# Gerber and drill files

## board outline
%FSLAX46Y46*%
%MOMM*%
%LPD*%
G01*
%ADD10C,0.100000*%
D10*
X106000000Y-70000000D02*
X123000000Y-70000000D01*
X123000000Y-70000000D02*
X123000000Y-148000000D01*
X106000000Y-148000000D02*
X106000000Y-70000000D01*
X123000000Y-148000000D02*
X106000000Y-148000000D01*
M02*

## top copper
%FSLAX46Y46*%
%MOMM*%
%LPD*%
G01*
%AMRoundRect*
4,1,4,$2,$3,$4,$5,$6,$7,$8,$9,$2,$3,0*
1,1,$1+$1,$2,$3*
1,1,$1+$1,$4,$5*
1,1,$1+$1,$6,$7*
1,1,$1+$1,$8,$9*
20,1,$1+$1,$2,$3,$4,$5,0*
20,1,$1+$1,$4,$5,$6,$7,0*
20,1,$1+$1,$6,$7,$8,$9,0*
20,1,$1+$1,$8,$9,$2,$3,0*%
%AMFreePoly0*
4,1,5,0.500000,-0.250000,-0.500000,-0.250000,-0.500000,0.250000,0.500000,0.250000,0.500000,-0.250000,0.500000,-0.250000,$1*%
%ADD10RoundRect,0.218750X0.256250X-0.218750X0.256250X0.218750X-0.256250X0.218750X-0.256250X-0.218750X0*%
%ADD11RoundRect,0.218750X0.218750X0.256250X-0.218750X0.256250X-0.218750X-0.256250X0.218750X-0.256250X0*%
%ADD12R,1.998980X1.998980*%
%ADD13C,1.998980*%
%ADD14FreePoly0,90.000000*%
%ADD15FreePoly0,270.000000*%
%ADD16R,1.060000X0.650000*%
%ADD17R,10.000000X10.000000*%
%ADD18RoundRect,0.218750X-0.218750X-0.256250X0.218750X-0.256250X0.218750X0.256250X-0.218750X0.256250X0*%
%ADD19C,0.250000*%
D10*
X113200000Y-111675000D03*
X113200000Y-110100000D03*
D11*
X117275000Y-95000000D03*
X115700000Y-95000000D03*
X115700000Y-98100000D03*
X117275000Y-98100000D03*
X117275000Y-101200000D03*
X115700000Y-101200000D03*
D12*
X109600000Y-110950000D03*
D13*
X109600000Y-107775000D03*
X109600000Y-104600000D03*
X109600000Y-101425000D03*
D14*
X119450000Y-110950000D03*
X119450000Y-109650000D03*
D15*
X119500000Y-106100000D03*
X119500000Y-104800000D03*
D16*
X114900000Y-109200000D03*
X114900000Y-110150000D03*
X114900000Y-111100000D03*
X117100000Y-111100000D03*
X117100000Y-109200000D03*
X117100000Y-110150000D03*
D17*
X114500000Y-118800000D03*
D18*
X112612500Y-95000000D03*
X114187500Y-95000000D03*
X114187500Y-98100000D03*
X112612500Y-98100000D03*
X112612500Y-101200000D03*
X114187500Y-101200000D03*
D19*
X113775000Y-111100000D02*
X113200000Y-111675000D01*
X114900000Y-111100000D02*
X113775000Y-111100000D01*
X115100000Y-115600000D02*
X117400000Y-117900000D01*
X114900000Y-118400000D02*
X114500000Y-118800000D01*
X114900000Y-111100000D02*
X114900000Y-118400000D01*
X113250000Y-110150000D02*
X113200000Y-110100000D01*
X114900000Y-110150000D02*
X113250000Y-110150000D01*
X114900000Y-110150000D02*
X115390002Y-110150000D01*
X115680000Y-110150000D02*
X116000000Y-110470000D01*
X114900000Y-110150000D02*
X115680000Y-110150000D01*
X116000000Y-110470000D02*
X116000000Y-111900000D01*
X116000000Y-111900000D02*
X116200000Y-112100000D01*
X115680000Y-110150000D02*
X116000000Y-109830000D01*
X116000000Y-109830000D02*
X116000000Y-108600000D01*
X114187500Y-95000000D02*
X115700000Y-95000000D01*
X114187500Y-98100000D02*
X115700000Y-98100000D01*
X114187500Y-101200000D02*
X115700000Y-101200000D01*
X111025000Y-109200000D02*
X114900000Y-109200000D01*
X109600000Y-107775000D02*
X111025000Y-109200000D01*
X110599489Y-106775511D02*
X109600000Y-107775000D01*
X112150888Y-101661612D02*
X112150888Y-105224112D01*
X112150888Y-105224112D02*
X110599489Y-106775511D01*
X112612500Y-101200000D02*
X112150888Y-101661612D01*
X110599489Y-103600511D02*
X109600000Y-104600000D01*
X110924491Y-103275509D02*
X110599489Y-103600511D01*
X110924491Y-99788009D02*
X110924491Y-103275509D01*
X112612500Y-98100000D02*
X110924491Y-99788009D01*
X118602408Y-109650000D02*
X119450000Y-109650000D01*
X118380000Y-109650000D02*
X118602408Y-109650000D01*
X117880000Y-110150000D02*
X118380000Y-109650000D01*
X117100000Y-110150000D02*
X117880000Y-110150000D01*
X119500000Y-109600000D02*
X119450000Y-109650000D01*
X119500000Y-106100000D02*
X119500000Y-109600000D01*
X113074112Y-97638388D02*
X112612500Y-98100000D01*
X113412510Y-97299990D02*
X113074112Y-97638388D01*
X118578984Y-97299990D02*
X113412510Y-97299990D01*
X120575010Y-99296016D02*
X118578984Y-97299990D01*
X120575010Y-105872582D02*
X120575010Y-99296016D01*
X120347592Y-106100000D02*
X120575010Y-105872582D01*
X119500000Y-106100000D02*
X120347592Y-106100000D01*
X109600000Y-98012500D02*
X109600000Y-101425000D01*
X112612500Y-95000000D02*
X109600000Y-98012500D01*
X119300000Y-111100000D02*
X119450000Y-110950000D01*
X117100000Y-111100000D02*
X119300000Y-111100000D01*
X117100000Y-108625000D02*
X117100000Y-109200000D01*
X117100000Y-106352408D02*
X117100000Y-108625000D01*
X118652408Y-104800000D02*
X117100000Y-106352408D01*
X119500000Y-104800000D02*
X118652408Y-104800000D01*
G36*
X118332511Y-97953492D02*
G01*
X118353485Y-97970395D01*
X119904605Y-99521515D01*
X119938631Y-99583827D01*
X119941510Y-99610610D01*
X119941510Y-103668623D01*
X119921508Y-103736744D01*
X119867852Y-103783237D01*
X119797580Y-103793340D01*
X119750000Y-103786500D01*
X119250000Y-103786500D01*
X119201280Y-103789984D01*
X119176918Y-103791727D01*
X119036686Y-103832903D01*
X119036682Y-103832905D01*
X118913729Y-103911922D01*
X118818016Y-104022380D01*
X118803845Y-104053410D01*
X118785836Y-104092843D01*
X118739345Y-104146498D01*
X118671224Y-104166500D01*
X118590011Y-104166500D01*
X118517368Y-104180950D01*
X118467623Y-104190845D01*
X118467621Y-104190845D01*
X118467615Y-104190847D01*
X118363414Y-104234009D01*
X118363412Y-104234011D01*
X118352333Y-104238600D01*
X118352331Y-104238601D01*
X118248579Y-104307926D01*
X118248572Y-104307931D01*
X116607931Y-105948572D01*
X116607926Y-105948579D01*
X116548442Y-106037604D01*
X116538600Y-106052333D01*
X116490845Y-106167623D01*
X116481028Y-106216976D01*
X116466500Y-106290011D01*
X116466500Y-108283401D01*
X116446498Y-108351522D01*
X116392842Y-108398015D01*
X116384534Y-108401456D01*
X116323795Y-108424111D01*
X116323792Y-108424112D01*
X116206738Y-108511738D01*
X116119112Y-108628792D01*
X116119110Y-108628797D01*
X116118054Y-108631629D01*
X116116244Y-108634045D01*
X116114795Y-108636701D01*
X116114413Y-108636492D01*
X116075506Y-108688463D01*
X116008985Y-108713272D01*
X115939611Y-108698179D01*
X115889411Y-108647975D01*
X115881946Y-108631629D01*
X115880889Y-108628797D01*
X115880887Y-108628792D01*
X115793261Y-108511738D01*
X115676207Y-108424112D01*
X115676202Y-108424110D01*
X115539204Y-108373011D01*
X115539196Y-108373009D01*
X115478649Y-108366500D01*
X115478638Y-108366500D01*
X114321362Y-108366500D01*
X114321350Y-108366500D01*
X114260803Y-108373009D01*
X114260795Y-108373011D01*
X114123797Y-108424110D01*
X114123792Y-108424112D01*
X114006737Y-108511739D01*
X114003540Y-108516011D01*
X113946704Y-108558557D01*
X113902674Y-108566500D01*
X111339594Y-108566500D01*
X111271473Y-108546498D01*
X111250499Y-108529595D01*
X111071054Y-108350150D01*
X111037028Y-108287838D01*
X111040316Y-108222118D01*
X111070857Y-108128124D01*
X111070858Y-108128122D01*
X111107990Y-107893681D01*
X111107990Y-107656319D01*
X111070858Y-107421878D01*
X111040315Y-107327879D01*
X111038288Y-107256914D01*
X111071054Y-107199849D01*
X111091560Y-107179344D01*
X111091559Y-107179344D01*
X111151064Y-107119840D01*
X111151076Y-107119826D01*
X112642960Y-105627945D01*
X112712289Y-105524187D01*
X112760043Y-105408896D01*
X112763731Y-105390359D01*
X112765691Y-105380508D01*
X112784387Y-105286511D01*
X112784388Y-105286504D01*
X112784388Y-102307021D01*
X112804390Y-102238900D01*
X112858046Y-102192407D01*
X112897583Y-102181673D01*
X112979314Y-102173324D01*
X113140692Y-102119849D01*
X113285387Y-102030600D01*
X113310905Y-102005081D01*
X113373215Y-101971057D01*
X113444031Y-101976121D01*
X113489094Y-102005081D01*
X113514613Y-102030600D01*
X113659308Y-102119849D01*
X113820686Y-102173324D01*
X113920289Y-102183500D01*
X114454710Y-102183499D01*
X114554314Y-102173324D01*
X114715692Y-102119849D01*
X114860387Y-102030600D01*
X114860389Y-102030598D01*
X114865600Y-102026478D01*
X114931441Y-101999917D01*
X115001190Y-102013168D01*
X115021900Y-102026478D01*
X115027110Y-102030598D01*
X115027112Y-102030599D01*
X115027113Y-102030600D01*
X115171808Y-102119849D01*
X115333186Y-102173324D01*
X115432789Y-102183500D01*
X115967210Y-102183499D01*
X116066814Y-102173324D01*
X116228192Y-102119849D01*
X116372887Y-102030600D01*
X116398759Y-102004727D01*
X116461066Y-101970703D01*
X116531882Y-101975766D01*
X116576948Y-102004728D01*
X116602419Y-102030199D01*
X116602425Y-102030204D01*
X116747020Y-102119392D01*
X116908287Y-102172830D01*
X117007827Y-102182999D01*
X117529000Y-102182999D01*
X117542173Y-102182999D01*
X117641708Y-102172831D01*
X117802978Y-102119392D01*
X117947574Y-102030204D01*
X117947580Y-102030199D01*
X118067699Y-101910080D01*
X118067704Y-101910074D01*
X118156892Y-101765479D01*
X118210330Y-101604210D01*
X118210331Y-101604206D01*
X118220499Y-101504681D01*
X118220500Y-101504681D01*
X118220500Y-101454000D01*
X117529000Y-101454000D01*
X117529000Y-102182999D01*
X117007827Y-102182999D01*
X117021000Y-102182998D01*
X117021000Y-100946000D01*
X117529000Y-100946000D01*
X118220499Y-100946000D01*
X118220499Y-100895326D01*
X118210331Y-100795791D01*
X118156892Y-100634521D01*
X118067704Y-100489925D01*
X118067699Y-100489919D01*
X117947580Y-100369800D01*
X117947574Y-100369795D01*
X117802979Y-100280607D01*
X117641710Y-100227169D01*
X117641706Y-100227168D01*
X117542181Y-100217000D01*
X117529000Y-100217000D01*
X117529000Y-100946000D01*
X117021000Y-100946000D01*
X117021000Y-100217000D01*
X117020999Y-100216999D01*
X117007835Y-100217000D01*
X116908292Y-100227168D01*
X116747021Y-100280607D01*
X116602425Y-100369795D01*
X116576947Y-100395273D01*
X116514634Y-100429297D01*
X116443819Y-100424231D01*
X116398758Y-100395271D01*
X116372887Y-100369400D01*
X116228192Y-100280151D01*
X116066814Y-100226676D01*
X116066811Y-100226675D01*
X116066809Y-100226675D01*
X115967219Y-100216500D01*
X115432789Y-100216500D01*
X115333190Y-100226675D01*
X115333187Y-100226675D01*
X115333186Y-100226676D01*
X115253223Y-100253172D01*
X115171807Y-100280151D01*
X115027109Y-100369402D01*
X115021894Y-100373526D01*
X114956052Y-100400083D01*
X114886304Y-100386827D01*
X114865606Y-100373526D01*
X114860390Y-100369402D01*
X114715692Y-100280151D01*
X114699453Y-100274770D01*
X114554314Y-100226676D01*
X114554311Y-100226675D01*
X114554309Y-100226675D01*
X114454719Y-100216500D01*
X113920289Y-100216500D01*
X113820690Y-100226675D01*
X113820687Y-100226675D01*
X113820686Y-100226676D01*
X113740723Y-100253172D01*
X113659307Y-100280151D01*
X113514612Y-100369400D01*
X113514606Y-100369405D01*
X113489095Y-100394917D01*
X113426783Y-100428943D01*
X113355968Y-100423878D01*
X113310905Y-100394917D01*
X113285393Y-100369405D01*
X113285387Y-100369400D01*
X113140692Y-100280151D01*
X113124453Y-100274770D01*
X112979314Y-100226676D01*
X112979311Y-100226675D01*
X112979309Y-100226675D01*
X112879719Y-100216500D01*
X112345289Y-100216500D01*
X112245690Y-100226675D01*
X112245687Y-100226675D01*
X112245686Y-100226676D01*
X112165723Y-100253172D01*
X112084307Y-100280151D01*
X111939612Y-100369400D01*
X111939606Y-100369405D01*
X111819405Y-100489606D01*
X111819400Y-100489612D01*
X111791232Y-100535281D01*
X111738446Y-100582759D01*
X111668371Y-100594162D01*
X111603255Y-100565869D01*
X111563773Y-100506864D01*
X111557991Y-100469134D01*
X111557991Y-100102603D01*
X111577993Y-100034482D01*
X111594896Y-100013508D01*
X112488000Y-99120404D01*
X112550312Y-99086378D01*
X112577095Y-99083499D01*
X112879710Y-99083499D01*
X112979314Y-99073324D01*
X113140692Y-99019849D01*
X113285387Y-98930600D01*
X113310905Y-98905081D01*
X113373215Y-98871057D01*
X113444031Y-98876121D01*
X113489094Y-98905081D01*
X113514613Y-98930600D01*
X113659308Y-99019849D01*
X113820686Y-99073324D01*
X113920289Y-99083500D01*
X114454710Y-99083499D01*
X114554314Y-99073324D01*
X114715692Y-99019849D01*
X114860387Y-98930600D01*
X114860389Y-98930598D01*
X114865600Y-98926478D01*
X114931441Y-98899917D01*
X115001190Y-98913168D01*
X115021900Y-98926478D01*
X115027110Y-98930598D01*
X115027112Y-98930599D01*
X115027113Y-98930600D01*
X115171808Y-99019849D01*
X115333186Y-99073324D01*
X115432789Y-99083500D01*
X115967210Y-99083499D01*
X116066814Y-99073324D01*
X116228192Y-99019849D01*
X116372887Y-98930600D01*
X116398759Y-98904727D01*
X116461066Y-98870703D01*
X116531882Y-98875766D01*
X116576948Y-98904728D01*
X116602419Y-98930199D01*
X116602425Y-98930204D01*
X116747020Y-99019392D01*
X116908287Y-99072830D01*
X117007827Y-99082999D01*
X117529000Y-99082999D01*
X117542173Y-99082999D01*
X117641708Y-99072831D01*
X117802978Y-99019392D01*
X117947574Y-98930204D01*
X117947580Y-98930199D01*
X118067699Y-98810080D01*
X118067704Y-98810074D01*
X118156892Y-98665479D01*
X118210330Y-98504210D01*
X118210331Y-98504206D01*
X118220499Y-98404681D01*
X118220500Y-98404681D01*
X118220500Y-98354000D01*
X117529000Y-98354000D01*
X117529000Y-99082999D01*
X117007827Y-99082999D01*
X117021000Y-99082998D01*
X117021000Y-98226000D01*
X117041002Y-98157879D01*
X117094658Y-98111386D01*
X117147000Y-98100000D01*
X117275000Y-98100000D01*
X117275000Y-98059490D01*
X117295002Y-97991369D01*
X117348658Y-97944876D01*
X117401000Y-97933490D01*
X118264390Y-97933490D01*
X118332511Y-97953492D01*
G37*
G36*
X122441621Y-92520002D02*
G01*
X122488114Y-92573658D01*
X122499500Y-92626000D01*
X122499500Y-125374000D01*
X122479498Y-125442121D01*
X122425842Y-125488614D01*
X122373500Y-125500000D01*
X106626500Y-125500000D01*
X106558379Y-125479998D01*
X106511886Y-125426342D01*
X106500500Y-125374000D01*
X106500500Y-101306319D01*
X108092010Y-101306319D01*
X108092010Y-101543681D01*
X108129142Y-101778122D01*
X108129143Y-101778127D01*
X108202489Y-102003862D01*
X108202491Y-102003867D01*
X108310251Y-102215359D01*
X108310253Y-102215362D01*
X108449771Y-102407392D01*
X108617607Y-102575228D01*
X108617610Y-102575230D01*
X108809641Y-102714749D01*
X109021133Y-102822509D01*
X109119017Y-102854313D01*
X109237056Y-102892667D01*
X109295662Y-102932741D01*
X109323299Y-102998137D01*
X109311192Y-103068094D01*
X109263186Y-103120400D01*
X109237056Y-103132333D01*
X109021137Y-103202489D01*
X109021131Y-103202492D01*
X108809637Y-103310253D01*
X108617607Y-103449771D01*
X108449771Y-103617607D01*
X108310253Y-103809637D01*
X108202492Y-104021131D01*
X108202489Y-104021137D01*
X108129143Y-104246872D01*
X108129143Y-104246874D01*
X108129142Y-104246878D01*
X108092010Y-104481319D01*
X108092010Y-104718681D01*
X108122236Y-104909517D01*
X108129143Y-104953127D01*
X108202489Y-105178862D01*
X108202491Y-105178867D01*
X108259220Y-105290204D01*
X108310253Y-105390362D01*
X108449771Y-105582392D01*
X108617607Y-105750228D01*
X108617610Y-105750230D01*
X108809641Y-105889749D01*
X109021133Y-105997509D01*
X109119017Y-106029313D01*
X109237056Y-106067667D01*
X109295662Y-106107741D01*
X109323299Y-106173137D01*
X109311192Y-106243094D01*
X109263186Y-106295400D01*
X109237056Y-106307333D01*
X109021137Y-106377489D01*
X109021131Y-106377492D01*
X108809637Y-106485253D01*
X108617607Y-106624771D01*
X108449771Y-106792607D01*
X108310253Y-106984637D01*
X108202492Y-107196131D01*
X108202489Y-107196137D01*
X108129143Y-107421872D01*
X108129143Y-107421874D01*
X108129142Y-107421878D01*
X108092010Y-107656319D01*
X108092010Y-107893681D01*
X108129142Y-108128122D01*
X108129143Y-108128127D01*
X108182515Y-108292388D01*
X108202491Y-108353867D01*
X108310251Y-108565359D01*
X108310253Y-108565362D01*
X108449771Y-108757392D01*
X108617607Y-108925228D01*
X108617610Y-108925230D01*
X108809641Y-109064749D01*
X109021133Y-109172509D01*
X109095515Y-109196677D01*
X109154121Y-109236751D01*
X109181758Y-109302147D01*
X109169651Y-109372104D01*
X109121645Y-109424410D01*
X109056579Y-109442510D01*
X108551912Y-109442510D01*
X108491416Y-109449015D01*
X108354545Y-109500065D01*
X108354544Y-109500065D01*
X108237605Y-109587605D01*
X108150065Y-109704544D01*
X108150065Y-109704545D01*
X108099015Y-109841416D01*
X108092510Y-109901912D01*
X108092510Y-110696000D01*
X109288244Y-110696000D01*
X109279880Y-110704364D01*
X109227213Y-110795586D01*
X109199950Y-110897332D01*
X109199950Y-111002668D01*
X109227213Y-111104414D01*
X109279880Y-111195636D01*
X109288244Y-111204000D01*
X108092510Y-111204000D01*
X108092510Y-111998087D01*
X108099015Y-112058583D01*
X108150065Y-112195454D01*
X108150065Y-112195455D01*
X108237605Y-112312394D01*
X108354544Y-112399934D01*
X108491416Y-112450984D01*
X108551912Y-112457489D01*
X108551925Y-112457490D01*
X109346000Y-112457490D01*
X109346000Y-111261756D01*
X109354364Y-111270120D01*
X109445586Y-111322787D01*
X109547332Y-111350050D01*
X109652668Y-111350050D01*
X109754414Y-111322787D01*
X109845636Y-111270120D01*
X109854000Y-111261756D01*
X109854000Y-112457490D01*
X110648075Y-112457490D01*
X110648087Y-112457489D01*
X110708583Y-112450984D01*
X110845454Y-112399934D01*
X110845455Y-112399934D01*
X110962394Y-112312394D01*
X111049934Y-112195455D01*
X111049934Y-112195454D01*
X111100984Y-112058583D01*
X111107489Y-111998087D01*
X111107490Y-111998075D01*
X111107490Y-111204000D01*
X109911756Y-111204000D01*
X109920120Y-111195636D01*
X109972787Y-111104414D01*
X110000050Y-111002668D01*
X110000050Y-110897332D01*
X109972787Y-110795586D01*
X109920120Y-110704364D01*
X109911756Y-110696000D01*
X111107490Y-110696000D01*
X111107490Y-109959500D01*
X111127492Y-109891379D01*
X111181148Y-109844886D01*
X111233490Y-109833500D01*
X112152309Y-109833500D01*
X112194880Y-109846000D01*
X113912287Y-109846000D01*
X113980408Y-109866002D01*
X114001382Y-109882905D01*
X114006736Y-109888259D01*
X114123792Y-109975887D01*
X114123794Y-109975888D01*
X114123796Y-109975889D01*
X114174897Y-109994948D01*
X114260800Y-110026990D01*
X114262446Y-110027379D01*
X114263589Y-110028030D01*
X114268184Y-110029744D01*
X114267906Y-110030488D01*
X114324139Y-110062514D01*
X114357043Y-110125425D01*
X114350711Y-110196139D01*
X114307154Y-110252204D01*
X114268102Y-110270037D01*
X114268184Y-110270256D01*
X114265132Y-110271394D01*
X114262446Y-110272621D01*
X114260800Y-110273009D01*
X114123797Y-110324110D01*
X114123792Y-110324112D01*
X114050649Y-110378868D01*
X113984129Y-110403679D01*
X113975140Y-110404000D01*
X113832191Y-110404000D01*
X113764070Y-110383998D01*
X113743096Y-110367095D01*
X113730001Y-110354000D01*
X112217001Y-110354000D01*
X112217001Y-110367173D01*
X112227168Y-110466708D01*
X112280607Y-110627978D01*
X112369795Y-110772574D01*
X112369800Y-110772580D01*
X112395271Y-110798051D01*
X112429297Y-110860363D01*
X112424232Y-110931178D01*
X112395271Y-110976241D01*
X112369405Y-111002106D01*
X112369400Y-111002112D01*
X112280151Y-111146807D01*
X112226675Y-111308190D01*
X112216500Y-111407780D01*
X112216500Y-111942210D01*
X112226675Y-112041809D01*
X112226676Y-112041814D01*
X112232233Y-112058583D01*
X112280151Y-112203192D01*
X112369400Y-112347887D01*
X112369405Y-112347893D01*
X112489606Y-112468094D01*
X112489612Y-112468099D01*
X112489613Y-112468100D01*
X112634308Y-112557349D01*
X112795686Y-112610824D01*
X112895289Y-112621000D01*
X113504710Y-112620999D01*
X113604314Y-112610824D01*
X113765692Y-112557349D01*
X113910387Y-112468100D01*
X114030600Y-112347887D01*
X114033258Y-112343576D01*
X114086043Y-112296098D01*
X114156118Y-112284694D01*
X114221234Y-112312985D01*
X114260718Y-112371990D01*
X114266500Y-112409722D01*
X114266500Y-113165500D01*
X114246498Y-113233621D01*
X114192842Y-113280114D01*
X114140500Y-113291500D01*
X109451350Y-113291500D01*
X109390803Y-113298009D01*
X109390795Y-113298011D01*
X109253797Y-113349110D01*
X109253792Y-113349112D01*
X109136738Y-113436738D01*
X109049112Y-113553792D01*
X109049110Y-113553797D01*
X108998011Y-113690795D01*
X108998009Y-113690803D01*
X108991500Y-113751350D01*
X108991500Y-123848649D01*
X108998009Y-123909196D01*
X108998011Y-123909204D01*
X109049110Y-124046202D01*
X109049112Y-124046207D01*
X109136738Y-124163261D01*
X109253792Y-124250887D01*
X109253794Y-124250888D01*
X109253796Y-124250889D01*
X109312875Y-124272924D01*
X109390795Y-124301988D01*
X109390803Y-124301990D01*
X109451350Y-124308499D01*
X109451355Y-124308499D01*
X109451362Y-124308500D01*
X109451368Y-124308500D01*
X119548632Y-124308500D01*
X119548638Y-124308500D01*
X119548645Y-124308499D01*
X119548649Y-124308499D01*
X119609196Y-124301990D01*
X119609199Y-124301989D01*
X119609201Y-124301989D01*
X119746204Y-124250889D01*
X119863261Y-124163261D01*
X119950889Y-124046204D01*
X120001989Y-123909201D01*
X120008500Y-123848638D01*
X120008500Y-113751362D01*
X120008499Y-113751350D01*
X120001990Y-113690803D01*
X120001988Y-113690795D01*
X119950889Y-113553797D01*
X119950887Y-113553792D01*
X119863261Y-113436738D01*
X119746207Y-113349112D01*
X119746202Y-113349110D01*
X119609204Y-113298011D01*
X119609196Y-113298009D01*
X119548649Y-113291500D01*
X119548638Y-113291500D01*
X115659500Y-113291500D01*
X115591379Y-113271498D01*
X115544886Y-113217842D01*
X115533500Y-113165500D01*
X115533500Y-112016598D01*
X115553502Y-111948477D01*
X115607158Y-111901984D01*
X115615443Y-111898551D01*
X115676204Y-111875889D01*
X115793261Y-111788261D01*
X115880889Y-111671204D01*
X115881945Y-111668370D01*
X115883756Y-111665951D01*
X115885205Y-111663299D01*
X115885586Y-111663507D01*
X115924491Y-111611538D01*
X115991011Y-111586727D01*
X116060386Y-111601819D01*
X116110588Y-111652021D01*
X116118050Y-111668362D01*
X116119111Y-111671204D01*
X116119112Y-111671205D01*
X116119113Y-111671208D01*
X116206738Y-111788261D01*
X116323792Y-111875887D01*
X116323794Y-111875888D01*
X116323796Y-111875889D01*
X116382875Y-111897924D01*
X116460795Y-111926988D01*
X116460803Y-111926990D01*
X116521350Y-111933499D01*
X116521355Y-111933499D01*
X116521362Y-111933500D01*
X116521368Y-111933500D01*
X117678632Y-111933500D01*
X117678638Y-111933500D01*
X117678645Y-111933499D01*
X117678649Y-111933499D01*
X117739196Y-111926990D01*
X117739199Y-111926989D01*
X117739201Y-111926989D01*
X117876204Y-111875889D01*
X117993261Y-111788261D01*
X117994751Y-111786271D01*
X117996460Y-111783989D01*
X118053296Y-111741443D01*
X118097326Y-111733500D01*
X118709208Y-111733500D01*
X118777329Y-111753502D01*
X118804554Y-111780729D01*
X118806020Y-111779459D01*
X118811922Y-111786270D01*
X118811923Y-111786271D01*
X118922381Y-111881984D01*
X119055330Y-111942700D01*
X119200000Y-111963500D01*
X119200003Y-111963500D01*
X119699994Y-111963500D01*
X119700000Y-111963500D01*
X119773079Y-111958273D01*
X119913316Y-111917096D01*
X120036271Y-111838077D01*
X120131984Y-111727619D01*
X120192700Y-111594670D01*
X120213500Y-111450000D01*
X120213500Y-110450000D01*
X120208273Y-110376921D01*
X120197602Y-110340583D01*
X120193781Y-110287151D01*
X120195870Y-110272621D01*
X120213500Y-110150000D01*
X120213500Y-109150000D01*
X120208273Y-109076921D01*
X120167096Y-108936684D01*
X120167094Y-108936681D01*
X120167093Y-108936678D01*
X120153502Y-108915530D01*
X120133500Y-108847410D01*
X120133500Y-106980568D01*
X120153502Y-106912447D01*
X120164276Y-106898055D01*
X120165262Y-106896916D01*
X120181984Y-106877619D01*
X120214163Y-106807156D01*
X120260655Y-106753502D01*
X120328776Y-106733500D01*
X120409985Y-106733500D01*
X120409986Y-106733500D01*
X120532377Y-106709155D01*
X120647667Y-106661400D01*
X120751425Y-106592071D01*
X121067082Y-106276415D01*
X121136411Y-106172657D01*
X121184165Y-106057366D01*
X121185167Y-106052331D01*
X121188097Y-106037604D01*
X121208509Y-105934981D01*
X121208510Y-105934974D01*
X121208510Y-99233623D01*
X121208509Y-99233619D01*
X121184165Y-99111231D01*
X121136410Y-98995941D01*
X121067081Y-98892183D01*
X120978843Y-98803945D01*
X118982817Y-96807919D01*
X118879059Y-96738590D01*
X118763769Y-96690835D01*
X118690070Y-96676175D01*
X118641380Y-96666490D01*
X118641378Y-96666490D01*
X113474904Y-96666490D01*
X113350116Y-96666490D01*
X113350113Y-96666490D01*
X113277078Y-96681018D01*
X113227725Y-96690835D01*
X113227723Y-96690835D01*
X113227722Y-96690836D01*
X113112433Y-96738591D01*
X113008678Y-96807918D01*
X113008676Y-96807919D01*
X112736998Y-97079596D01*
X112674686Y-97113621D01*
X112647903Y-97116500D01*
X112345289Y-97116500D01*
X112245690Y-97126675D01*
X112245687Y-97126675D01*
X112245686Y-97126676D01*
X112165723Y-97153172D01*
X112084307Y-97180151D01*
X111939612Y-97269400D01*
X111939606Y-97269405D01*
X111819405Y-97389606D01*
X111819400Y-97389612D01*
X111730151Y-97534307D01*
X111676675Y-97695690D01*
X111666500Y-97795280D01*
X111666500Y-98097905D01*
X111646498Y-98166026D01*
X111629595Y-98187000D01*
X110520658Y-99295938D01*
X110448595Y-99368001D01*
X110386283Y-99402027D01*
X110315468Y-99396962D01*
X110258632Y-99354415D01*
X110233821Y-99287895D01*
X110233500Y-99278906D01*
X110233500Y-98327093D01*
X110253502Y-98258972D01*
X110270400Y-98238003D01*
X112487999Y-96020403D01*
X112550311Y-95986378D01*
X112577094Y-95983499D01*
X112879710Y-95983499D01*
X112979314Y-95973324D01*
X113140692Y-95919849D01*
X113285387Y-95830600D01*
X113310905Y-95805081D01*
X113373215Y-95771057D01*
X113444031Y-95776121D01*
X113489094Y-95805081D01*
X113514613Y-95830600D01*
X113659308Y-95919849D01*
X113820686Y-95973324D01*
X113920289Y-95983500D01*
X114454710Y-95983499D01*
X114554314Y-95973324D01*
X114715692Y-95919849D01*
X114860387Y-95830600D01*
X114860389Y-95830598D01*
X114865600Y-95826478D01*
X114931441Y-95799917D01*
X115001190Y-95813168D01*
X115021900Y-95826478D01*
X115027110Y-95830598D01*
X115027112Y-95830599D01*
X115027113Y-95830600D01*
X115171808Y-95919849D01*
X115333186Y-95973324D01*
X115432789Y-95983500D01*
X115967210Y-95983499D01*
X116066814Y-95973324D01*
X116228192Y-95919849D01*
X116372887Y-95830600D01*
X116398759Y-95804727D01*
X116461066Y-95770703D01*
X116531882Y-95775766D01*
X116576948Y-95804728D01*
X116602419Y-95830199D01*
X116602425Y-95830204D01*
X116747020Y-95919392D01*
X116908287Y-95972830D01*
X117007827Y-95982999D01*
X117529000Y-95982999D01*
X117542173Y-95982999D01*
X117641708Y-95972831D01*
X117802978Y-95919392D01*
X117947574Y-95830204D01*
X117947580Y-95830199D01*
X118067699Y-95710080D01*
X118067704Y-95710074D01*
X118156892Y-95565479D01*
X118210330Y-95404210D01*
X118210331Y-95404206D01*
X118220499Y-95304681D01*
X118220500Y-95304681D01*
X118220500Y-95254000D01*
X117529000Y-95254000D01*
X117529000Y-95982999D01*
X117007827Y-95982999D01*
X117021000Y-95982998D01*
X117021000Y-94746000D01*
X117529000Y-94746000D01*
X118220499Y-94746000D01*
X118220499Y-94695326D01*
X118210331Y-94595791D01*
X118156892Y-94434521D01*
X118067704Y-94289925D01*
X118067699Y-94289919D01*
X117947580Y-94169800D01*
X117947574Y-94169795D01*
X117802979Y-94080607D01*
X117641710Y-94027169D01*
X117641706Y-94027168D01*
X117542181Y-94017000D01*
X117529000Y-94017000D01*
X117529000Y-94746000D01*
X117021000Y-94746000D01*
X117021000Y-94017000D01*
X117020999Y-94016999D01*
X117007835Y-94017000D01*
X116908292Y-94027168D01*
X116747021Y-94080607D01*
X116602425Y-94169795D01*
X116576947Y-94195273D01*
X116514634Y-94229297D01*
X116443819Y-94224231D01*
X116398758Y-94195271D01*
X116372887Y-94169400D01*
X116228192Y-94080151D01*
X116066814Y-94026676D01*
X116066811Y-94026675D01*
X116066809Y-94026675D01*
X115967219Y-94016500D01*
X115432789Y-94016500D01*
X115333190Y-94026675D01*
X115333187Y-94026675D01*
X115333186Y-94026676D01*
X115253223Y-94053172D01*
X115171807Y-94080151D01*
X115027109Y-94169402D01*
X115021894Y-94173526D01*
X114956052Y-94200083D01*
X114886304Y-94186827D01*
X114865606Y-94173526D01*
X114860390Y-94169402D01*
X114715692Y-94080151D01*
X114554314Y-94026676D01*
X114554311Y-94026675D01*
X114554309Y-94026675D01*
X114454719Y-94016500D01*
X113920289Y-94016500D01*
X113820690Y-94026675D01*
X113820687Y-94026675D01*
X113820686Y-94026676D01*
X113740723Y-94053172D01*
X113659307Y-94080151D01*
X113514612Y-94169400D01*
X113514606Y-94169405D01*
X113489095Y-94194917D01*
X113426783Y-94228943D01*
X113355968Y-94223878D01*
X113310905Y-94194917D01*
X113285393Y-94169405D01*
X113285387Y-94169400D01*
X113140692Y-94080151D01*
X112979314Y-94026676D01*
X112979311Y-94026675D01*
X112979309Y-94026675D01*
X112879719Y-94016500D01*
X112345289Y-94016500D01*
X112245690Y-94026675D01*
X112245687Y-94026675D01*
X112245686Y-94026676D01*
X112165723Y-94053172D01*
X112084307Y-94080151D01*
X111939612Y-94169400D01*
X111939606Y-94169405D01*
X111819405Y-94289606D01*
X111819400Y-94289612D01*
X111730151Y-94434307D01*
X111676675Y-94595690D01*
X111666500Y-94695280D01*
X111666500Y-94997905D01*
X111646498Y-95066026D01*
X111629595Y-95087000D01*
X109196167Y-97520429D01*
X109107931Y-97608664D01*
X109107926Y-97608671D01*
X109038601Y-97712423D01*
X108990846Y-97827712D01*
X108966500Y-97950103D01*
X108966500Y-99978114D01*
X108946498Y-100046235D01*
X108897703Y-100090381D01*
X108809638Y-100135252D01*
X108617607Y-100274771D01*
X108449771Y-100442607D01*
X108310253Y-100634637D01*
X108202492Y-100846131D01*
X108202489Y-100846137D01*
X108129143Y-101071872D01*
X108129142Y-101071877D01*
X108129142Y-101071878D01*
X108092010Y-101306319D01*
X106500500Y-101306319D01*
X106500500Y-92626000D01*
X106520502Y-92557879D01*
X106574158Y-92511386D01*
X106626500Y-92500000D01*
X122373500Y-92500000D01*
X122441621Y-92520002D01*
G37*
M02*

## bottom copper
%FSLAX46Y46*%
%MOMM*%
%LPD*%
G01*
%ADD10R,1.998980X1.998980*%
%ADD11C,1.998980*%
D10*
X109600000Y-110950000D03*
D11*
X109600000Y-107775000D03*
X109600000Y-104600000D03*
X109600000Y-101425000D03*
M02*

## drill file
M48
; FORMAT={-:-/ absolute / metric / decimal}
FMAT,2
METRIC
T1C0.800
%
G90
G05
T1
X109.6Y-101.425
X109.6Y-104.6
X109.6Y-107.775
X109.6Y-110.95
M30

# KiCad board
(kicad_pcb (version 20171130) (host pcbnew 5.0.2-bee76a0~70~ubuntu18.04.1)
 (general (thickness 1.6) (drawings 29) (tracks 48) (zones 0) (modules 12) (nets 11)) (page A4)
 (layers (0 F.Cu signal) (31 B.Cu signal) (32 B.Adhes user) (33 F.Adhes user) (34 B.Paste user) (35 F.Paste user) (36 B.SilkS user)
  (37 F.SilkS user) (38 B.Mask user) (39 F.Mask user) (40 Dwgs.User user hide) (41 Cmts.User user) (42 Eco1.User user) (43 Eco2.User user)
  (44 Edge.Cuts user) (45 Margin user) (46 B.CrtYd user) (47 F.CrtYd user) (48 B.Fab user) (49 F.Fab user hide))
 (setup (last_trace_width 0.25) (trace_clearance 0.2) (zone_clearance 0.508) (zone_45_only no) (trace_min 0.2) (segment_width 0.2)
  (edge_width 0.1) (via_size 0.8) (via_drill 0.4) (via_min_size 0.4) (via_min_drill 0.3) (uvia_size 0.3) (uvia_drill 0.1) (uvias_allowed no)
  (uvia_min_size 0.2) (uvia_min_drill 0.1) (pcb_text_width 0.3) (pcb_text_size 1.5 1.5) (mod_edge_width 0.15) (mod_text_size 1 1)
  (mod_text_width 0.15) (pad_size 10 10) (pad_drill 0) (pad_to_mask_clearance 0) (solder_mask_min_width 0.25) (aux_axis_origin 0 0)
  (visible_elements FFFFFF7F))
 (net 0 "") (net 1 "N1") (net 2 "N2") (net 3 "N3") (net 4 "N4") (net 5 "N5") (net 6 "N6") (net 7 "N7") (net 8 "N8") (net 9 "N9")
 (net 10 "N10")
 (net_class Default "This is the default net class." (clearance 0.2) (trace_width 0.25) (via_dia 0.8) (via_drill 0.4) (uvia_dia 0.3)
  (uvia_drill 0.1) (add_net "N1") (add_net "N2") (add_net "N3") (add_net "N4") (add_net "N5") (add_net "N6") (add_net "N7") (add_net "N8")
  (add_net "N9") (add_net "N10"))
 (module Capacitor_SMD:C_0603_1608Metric (layer F.Cu) (at 113.2 110.8875 90)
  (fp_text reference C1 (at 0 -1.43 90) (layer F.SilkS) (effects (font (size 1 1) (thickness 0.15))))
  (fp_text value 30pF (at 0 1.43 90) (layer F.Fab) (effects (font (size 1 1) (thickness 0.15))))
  (pad 1 smd roundrect (at -0.7875 0 90) (size 0.875 0.95) (layers F.Cu F.Paste F.Mask) (roundrect_rratio 0.25) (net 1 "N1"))
  (pad 2 smd roundrect (at 0.7875 0 90) (size 0.875 0.95) (layers F.Cu F.Paste F.Mask) (roundrect_rratio 0.25) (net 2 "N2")))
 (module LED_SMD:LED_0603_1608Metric (layer F.Cu) (at 116.4875 95 180)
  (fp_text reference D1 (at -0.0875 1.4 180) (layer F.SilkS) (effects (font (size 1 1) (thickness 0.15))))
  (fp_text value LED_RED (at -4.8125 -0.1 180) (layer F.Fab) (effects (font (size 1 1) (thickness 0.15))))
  (pad 1 smd roundrect (at -0.7875 0 180) (size 0.875 0.95) (layers F.Cu F.Paste F.Mask) (roundrect_rratio 0.25) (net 2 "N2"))
  (pad 2 smd roundrect (at 0.7875 0 180) (size 0.875 0.95) (layers F.Cu F.Paste F.Mask) (roundrect_rratio 0.25) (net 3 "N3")))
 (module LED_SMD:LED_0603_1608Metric (layer F.Cu) (at 116.4875 98.1 180)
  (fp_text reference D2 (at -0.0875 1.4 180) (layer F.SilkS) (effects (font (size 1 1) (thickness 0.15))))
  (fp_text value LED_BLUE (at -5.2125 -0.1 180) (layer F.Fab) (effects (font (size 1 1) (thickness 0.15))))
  (pad 2 smd roundrect (at 0.7875 0 180) (size 0.875 0.95) (layers F.Cu F.Paste F.Mask) (roundrect_rratio 0.25) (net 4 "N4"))
  (pad 1 smd roundrect (at -0.7875 0 180) (size 0.875 0.95) (layers F.Cu F.Paste F.Mask) (roundrect_rratio 0.25) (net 2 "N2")))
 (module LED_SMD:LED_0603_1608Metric (layer F.Cu) (at 116.4875 101.2 180)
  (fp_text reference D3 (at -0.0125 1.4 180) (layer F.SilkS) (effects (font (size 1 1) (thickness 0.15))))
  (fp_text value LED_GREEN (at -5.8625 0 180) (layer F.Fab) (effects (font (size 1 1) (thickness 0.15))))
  (pad 1 smd roundrect (at -0.7875 0 180) (size 0.875 0.95) (layers F.Cu F.Paste F.Mask) (roundrect_rratio 0.25) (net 2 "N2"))
  (pad 2 smd roundrect (at 0.7875 0 180) (size 0.875 0.95) (layers F.Cu F.Paste F.Mask) (roundrect_rratio 0.25) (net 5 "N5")))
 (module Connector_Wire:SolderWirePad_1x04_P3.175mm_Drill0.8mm (layer F.Cu) (at 109.6 110.95 90)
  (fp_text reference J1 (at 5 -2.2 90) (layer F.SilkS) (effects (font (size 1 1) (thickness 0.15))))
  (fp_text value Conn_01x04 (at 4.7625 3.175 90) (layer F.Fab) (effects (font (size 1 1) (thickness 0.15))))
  (pad 1 thru_hole rect (at 0 0 90) (size 1.99898 1.99898) (drill 0.8001) (layers *.Cu *.Mask) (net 2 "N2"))
  (pad 2 thru_hole circle (at 3.175 0 90) (size 1.99898 1.99898) (drill 0.8001) (layers *.Cu *.Mask) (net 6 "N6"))
  (pad 3 thru_hole circle (at 6.35 0 90) (size 1.99898 1.99898) (drill 0.8001) (layers *.Cu *.Mask) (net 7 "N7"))
  (pad 4 thru_hole circle (at 9.525 0 90) (size 1.99898 1.99898) (drill 0.8001) (layers *.Cu *.Mask) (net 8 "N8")))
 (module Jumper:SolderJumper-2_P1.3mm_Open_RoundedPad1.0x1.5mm (layer F.Cu) (at 119.45 110.3 90)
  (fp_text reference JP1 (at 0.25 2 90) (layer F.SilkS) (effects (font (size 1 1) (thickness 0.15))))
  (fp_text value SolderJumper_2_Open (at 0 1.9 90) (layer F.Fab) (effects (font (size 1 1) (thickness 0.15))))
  (pad 1 smd custom (at -0.65 0 90) (size 1 0.5) (layers F.Cu F.Mask) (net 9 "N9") (zone_connect 0)
   (options (clearance outline) (anchor rect)) (primitives))
  (pad 2 smd custom (at 0.65 0 90) (size 1 0.5) (layers F.Cu F.Mask) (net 7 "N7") (zone_connect 0)
   (options (clearance outline) (anchor rect)) (primitives)))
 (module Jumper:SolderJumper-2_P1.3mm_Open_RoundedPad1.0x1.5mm (layer F.Cu) (at 119.5 105.45 270)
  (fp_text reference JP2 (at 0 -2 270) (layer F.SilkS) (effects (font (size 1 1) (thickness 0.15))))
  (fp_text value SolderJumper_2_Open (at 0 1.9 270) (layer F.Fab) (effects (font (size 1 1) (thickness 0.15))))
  (pad 2 smd custom (at 0.65 0 270) (size 1 0.5) (layers F.Cu F.Mask) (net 7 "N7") (zone_connect 0)
   (options (clearance outline) (anchor rect)) (primitives))
  (pad 1 smd custom (at -0.65 0 270) (size 1 0.5) (layers F.Cu F.Mask) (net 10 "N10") (zone_connect 0)
   (options (clearance outline) (anchor rect)) (primitives)))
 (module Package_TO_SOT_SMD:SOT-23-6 (layer F.Cu) (at 116 110.15)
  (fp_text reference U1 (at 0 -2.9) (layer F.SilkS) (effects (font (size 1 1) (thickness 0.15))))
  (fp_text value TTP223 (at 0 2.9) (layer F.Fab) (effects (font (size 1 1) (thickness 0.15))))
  (pad 1 smd rect (at -1.1 -0.95) (size 1.06 0.65) (layers F.Cu F.Paste F.Mask) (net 6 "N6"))
  (pad 2 smd rect (at -1.1 0) (size 1.06 0.65) (layers F.Cu F.Paste F.Mask) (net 2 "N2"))
  (pad 3 smd rect (at -1.1 0.95) (size 1.06 0.65) (layers F.Cu F.Paste F.Mask) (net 1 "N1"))
  (pad 4 smd rect (at 1.1 0.95) (size 1.06 0.65) (layers F.Cu F.Paste F.Mask) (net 9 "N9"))
  (pad 6 smd rect (at 1.1 -0.95) (size 1.06 0.65) (layers F.Cu F.Paste F.Mask) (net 10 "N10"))
  (pad 5 smd rect (at 1.1 0) (size 1.06 0.65) (layers F.Cu F.Paste F.Mask) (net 7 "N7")))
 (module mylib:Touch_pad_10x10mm (layer F.Cu) (at 114.5 118.8)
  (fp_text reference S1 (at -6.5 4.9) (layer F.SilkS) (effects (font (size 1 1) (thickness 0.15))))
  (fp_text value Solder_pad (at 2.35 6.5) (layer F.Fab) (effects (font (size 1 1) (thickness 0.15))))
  (pad 1 smd rect (at 0 0) (size 10 10) (layers F.Cu F.Paste F.Mask) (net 1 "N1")))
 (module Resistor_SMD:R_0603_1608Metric (layer F.Cu) (at 113.4 95)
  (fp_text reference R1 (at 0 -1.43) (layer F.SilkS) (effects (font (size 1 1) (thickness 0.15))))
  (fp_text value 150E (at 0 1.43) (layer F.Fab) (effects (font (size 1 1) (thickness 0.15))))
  (pad 1 smd roundrect (at -0.7875 0) (size 0.875 0.95) (layers F.Cu F.Paste F.Mask) (roundrect_rratio 0.25) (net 8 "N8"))
  (pad 2 smd roundrect (at 0.7875 0) (size 0.875 0.95) (layers F.Cu F.Paste F.Mask) (roundrect_rratio 0.25) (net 3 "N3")))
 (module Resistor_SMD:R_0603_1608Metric (layer F.Cu) (at 113.4 98.1)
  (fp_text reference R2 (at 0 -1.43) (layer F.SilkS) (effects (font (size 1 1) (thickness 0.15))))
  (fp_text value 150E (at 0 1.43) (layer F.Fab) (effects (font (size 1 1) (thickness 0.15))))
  (pad 2 smd roundrect (at 0.7875 0) (size 0.875 0.95) (layers F.Cu F.Paste F.Mask) (roundrect_rratio 0.25) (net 4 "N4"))
  (pad 1 smd roundrect (at -0.7875 0) (size 0.875 0.95) (layers F.Cu F.Paste F.Mask) (roundrect_rratio 0.25) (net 7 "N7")))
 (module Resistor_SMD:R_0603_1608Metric (layer F.Cu) (at 113.4 101.2)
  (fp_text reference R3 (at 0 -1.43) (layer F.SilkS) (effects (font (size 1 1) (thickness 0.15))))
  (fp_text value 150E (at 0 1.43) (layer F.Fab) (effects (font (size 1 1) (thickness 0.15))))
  (pad 1 smd roundrect (at -0.7875 0) (size 0.875 0.95) (layers F.Cu F.Paste F.Mask) (roundrect_rratio 0.25) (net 6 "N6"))
  (pad 2 smd roundrect (at 0.7875 0) (size 0.875 0.95) (layers F.Cu F.Paste F.Mask) (roundrect_rratio 0.25) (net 5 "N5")))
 (gr_line (start 106 70) (end 123 70) (layer Edge.Cuts) (width 0.1))
 (gr_line (start 123 70) (end 123 148) (layer Edge.Cuts) (width 0.1))
 (gr_line (start 106 148) (end 106 70) (layer Edge.Cuts) (width 0.1))
 (gr_line (start 123 148) (end 106 148) (layer Edge.Cuts) (width 0.1))
 (segment (start 113.775 111.1) (end 113.2 111.675) (width 0.25) (layer F.Cu) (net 1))
 (segment (start 114.9 111.1) (end 113.775 111.1) (width 0.25) (layer F.Cu) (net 1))
 (segment (start 115.1 115.6) (end 117.4 117.9) (width 0.25) (layer F.Cu) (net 1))
 (segment (start 114.9 118.4) (end 114.5 118.8) (width 0.25) (layer F.Cu) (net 1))
 (segment (start 114.9 111.1) (end 114.9 118.4) (width 0.25) (layer F.Cu) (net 1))
 (segment (start 113.25 110.15) (end 113.2 110.1) (width 0.25) (layer F.Cu) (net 2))
 (segment (start 114.9 110.15) (end 113.25 110.15) (width 0.25) (layer F.Cu) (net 2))
 (segment (start 114.9 110.15) (end 115.390002 110.15) (width 0.25) (layer F.Cu) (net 2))
 (segment (start 115.68 110.15) (end 116 110.47) (width 0.25) (layer F.Cu) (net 2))
 (segment (start 114.9 110.15) (end 115.68 110.15) (width 0.25) (layer F.Cu) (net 2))
 (segment (start 116 110.47) (end 116 111.9) (width 0.25) (layer F.Cu) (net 2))
 (segment (start 116 111.9) (end 116.2 112.1) (width 0.25) (layer F.Cu) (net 2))
 (segment (start 115.68 110.15) (end 116 109.83) (width 0.25) (layer F.Cu) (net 2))
 (segment (start 116 109.83) (end 116 108.6) (width 0.25) (layer F.Cu) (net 2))
 (segment (start 114.1875 95) (end 115.7 95) (width 0.25) (layer F.Cu) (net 3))
 (segment (start 114.1875 98.1) (end 115.7 98.1) (width 0.25) (layer F.Cu) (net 4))
 (segment (start 114.1875 101.2) (end 115.7 101.2) (width 0.25) (layer F.Cu) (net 5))
 (segment (start 111.025 109.2) (end 114.9 109.2) (width 0.25) (layer F.Cu) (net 6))
 (segment (start 109.6 107.775) (end 111.025 109.2) (width 0.25) (layer F.Cu) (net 6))
 (segment (start 110.599489 106.775511) (end 109.6 107.775) (width 0.25) (layer F.Cu) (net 6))
 (segment (start 112.150888 101.661612) (end 112.150888 105.224112) (width 0.25) (layer F.Cu) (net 6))
 (segment (start 112.150888 105.224112) (end 110.599489 106.775511) (width 0.25) (layer F.Cu) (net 6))
 (segment (start 112.6125 101.2) (end 112.150888 101.661612) (width 0.25) (layer F.Cu) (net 6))
 (segment (start 110.599489 103.600511) (end 109.6 104.6) (width 0.25) (layer F.Cu) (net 7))
 (segment (start 110.924491 103.275509) (end 110.599489 103.600511) (width 0.25) (layer F.Cu) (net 7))
 (segment (start 110.924491 99.788009) (end 110.924491 103.275509) (width 0.25) (layer F.Cu) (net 7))
 (segment (start 112.6125 98.1) (end 110.924491 99.788009) (width 0.25) (layer F.Cu) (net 7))
 (segment (start 118.602408 109.65) (end 119.45 109.65) (width 0.25) (layer F.Cu) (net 7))
 (segment (start 118.38 109.65) (end 118.602408 109.65) (width 0.25) (layer F.Cu) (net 7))
 (segment (start 117.88 110.15) (end 118.38 109.65) (width 0.25) (layer F.Cu) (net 7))
 (segment (start 117.1 110.15) (end 117.88 110.15) (width 0.25) (layer F.Cu) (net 7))
 (segment (start 119.5 109.6) (end 119.45 109.65) (width 0.25) (layer F.Cu) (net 7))
 (segment (start 119.5 106.1) (end 119.5 109.6) (width 0.25) (layer F.Cu) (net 7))
 (segment (start 113.074112 97.638388) (end 112.6125 98.1) (width 0.25) (layer F.Cu) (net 7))
 (segment (start 113.41251 97.29999) (end 113.074112 97.638388) (width 0.25) (layer F.Cu) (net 7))
 (segment (start 118.578984 97.29999) (end 113.41251 97.29999) (width 0.25) (layer F.Cu) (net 7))
 (segment (start 120.57501 99.296016) (end 118.578984 97.29999) (width 0.25) (layer F.Cu) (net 7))
 (segment (start 120.57501 105.872582) (end 120.57501 99.296016) (width 0.25) (layer F.Cu) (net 7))
 (segment (start 120.347592 106.1) (end 120.57501 105.872582) (width 0.25) (layer F.Cu) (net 7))
 (segment (start 119.5 106.1) (end 120.347592 106.1) (width 0.25) (layer F.Cu) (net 7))
 (segment (start 109.6 98.0125) (end 109.6 101.425) (width 0.25) (layer F.Cu) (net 8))
 (segment (start 112.6125 95) (end 109.6 98.0125) (width 0.25) (layer F.Cu) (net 8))
 (segment (start 119.3 111.1) (end 119.45 110.95) (width 0.25) (layer F.Cu) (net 9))
 (segment (start 117.1 111.1) (end 119.3 111.1) (width 0.25) (layer F.Cu) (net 9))
 (segment (start 117.1 108.625) (end 117.1 109.2) (width 0.25) (layer F.Cu) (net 10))
 (segment (start 117.1 106.352408) (end 117.1 108.625) (width 0.25) (layer F.Cu) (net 10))
 (segment (start 118.652408 104.8) (end 117.1 106.352408) (width 0.25) (layer F.Cu) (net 10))
 (segment (start 119.5 104.8) (end 118.652408 104.8) (width 0.25) (layer F.Cu) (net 10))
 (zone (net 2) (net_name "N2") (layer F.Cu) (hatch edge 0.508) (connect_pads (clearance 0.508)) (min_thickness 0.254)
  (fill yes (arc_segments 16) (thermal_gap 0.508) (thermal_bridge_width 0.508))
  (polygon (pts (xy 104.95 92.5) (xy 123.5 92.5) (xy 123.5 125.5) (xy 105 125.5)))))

